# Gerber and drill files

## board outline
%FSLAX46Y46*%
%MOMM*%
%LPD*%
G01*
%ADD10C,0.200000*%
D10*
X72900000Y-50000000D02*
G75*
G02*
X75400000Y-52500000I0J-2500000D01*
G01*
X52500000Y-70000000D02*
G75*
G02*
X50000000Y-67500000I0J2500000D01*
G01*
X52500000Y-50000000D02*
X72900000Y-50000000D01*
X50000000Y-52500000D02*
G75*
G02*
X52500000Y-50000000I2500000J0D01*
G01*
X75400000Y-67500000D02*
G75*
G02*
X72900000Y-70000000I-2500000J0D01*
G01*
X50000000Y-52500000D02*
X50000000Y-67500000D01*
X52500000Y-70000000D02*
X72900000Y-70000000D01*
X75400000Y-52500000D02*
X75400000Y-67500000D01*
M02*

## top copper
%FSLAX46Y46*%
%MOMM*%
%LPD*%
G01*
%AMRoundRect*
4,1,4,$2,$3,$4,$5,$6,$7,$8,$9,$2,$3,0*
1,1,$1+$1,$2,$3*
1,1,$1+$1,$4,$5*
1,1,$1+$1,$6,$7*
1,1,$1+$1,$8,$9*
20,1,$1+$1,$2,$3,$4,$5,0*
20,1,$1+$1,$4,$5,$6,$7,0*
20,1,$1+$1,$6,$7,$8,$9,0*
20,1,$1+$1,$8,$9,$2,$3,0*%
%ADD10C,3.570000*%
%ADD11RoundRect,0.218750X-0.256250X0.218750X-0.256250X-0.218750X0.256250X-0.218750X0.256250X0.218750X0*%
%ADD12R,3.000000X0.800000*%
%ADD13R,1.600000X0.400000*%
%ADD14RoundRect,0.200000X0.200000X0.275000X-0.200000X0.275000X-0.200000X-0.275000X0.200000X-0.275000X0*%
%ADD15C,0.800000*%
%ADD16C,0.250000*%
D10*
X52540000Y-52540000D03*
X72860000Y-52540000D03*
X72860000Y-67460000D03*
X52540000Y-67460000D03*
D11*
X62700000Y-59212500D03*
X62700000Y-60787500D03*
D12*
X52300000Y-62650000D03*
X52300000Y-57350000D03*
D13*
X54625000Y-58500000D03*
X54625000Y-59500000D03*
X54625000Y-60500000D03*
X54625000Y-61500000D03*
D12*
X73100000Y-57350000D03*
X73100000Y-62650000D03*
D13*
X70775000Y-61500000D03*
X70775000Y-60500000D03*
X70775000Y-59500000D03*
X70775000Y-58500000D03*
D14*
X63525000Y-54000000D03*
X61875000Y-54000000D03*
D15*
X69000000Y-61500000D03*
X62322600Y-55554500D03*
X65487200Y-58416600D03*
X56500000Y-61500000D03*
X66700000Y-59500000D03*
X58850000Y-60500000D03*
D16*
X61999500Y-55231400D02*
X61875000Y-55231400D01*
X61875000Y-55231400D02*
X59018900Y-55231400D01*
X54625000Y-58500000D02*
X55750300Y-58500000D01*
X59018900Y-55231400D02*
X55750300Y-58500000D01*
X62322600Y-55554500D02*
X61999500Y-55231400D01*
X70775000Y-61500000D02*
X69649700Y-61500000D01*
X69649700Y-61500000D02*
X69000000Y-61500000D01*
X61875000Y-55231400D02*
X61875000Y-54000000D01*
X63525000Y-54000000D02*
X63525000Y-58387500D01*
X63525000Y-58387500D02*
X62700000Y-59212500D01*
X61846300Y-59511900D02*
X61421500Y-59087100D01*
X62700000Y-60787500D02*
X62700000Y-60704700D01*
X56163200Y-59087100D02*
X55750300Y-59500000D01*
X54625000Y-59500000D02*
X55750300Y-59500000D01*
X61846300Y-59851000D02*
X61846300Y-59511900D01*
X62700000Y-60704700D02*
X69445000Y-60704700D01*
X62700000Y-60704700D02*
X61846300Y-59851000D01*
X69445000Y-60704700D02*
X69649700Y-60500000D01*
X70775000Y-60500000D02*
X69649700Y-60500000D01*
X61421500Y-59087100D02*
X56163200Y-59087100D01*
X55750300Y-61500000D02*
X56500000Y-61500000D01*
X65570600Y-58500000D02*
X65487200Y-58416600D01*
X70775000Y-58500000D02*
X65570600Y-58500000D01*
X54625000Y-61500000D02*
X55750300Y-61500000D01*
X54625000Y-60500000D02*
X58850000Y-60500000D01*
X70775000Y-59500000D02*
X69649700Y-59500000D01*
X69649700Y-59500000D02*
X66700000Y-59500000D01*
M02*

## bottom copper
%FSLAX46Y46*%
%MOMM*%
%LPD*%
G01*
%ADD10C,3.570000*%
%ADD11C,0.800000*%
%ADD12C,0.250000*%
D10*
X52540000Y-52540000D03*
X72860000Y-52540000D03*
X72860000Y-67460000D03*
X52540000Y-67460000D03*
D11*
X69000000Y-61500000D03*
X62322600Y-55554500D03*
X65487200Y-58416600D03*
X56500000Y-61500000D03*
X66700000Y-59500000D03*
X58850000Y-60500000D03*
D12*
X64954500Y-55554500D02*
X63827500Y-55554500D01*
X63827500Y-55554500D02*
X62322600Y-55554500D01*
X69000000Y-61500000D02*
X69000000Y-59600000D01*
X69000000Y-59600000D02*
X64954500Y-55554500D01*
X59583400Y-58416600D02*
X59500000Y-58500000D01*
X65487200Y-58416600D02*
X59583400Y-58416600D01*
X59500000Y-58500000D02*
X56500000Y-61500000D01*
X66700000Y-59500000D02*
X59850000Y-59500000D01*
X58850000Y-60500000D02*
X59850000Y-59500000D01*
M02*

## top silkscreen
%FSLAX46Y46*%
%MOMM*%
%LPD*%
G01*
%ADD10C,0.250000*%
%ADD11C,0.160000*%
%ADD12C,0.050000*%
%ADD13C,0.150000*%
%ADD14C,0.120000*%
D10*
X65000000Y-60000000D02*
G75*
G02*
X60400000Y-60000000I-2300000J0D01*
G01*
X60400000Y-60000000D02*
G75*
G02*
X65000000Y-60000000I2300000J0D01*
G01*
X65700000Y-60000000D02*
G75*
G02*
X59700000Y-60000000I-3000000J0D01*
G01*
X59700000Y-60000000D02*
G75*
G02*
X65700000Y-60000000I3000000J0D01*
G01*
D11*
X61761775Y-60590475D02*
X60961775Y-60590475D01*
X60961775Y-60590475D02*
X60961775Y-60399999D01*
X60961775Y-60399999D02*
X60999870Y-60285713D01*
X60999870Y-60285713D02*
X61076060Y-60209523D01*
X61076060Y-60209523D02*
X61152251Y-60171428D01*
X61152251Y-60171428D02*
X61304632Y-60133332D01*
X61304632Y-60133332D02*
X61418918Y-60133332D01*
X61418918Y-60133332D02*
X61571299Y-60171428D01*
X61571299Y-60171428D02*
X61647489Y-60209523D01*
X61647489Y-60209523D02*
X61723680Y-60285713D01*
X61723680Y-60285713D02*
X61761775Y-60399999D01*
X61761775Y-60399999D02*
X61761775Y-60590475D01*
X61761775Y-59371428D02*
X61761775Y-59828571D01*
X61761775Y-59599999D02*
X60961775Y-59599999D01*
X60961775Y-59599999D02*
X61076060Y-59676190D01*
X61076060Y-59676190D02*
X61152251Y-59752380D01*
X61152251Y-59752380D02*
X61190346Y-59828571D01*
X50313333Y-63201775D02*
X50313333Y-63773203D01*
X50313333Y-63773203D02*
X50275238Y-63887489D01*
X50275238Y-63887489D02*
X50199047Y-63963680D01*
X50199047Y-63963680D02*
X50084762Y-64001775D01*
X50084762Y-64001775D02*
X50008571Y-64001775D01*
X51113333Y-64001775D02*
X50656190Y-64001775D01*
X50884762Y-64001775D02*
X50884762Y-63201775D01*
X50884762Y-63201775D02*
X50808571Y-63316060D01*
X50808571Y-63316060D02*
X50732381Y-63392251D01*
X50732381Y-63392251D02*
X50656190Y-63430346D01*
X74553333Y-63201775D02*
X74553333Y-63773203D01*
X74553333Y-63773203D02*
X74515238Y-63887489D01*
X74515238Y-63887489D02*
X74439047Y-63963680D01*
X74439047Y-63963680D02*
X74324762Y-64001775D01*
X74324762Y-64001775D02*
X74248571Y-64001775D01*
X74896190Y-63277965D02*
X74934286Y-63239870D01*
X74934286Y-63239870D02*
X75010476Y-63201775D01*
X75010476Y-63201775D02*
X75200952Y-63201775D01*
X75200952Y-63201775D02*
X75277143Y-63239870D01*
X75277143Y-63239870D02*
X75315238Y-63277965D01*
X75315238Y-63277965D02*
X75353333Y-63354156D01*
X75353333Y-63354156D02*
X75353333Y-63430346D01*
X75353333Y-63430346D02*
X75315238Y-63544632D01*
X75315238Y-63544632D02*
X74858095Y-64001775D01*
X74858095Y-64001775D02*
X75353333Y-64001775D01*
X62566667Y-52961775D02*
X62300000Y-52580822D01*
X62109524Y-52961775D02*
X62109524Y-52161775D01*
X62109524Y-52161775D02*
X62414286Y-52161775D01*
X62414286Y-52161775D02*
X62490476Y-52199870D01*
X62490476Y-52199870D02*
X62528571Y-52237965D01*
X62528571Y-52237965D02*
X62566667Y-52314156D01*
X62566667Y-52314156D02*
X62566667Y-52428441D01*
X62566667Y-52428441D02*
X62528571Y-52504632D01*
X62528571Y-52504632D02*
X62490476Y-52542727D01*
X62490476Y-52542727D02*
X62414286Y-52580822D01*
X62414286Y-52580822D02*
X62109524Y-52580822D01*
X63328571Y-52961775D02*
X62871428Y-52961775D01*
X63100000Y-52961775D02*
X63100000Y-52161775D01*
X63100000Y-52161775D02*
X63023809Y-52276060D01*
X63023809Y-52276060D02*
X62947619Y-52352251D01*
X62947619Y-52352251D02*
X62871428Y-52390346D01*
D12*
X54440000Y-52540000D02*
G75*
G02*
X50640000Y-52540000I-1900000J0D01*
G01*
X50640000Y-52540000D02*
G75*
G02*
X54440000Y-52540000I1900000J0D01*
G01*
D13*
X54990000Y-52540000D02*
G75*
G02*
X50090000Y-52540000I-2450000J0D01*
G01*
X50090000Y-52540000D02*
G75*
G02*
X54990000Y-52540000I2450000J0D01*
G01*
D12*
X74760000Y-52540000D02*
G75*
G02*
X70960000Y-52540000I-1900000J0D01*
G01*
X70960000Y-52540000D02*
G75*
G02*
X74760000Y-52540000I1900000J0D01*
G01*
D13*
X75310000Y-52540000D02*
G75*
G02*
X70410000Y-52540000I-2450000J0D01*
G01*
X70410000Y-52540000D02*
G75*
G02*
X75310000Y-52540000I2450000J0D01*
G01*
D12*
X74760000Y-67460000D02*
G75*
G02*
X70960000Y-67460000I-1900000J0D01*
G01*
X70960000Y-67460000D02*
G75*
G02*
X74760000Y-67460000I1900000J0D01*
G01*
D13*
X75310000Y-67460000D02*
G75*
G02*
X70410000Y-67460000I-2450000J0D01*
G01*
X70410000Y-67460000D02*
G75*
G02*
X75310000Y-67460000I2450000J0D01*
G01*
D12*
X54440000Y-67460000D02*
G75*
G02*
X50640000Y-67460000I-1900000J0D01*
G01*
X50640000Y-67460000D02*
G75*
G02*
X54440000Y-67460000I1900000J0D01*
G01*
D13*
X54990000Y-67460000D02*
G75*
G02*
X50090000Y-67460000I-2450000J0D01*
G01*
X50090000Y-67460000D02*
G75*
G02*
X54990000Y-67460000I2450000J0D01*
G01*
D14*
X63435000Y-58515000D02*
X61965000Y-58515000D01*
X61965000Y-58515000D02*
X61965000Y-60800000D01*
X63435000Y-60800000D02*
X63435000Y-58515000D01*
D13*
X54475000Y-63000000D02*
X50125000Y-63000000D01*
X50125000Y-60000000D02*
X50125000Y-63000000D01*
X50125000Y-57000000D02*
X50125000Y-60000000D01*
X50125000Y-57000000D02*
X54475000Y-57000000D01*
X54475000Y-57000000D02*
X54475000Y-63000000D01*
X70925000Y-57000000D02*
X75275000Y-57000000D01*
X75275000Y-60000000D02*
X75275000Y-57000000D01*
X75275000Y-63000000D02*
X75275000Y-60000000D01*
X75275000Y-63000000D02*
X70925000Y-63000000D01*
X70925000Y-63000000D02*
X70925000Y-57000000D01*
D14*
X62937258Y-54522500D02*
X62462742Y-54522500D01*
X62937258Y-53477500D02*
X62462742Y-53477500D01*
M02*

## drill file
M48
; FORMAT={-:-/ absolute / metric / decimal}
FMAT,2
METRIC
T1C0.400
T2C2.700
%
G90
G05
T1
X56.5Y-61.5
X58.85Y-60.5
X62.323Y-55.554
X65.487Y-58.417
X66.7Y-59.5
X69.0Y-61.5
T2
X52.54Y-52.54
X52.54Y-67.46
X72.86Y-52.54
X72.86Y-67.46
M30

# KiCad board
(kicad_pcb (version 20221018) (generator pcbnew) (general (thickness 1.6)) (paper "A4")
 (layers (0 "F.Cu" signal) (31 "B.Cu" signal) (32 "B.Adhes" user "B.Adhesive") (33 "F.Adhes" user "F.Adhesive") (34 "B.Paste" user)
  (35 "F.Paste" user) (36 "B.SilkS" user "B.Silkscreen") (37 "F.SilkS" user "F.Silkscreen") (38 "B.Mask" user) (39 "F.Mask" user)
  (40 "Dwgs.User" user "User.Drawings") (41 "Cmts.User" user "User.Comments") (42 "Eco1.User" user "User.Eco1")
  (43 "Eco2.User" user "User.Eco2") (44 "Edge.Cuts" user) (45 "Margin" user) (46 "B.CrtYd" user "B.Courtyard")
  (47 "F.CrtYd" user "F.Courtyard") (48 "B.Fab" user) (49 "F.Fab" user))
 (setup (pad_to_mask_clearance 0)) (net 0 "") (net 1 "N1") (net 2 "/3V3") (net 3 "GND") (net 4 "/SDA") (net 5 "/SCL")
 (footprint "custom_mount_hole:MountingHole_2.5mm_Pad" (layer "F.Cu") (at 52.54 52.54)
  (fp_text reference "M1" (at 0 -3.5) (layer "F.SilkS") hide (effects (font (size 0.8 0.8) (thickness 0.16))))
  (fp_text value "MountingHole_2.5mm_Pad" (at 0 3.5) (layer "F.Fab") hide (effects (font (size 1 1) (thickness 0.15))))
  (fp_circle (center 0 0) (end 1.9 0) (stroke (width 0.05) (type solid)) (fill none) (layer "F.SilkS"))
  (fp_circle (center 0 0) (end 2.45 0) (stroke (width 0.15) (type solid)) (fill none) (layer "F.SilkS"))
  (pad "~" thru_hole circle (at 0 0) (size 3.57 3.57) (drill 2.7) (layers "*.Cu" "*.Mask")))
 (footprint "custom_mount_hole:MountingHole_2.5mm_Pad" (layer "F.Cu") (at 72.86 52.54)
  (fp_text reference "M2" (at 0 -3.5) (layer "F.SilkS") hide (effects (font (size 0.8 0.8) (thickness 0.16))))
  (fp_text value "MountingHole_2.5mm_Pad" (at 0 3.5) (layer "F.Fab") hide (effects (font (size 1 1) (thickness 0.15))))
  (fp_circle (center 0 0) (end 1.9 0) (stroke (width 0.05) (type solid)) (fill none) (layer "F.SilkS"))
  (fp_circle (center 0 0) (end 2.45 0) (stroke (width 0.15) (type solid)) (fill none) (layer "F.SilkS"))
  (pad "~" thru_hole circle (at 0 0) (size 3.57 3.57) (drill 2.7) (layers "*.Cu" "*.Mask")))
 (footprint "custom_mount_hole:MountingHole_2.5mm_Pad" (layer "F.Cu") (at 72.86 67.46)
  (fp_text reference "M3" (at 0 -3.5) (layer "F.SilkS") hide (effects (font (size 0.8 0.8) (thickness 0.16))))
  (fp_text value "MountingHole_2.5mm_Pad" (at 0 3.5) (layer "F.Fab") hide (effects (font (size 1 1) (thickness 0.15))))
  (fp_circle (center 0 0) (end 1.9 0) (stroke (width 0.05) (type solid)) (fill none) (layer "F.SilkS"))
  (fp_circle (center 0 0) (end 2.45 0) (stroke (width 0.15) (type solid)) (fill none) (layer "F.SilkS"))
  (pad "~" thru_hole circle (at 0 0) (size 3.57 3.57) (drill 2.7) (layers "*.Cu" "*.Mask")))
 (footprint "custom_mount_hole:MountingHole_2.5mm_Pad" (layer "F.Cu") (at 52.54 67.46)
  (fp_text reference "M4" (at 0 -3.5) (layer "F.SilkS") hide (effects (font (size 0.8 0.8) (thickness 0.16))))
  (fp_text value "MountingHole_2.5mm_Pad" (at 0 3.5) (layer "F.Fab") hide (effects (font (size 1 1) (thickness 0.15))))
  (fp_circle (center 0 0) (end 1.9 0) (stroke (width 0.05) (type solid)) (fill none) (layer "F.SilkS"))
  (fp_circle (center 0 0) (end 2.45 0) (stroke (width 0.15) (type solid)) (fill none) (layer "F.SilkS"))
  (pad "~" thru_hole circle (at 0 0) (size 3.57 3.57) (drill 2.7) (layers "*.Cu" "*.Mask")))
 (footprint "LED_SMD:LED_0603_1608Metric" (layer "F.Cu") (at 62.7 60 -90)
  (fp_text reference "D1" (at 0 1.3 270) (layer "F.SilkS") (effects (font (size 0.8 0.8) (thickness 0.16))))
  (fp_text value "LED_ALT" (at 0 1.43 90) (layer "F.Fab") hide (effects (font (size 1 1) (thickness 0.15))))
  (fp_line (start -1.485 -0.735) (end -1.485 0.735) (stroke (width 0.12) (type solid)) (layer "F.SilkS"))
  (fp_line (start -1.485 0.735) (end 0.8 0.735) (stroke (width 0.12) (type solid)) (layer "F.SilkS"))
  (fp_line (start 0.8 -0.735) (end -1.485 -0.735) (stroke (width 0.12) (type solid)) (layer "F.SilkS"))
  (pad "1" smd roundrect (at -0.7875 0 270) (size 0.875 0.95) (layers "F.Cu" "F.Paste" "F.Mask") (roundrect_rratio 0.25) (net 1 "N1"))
  (pad "2" smd roundrect (at 0.7875 0 270) (size 0.875 0.95) (layers "F.Cu" "F.Paste" "F.Mask") (roundrect_rratio 0.25) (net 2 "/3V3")))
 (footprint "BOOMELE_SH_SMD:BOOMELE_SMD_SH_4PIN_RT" (layer "F.Cu") (at 52.78 60 90)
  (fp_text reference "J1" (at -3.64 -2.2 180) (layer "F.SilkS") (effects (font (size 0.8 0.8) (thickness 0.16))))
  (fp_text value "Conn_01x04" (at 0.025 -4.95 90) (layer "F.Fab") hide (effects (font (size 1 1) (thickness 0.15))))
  (fp_line (start -3 1.695) (end -3 -2.655) (stroke (width 0.15) (type solid)) (layer "F.SilkS"))
  (fp_line (start 0 -2.655) (end -3 -2.655) (stroke (width 0.15) (type solid)) (layer "F.SilkS"))
  (fp_line (start 3 -2.655) (end 0 -2.655) (stroke (width 0.15) (type solid)) (layer "F.SilkS"))
  (fp_line (start 3 -2.655) (end 3 1.695) (stroke (width 0.15) (type solid)) (layer "F.SilkS"))
  (fp_line (start 3 1.695) (end -3 1.695) (stroke (width 0.15) (type solid)) (layer "F.SilkS"))
  (pad "" smd rect (at -2.65 -0.48 270) (size 0.8 3) (layers "F.Cu" "F.Paste" "F.Mask"))
  (pad "" smd rect (at 2.65 -0.48 270) (size 0.8 3) (layers "F.Cu" "F.Paste" "F.Mask"))
  (pad "1" smd rect (at 1.5 1.845 270) (size 0.4 1.6) (layers "F.Cu" "F.Paste" "F.Mask") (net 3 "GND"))
  (pad "2" smd rect (at 0.5 1.845 270) (size 0.4 1.6) (layers "F.Cu" "F.Paste" "F.Mask") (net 2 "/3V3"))
  (pad "3" smd rect (at -0.5 1.845 270) (size 0.4 1.6) (layers "F.Cu" "F.Paste" "F.Mask") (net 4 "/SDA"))
  (pad "4" smd rect (at -1.5 1.845 270) (size 0.4 1.6) (layers "F.Cu" "F.Paste" "F.Mask") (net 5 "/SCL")))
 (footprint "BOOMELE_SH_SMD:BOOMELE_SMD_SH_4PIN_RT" (layer "F.Cu") (at 72.62 60 -90)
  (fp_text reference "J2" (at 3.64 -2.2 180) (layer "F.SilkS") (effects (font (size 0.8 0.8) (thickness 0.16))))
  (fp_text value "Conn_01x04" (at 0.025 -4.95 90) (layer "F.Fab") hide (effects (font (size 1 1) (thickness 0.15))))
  (fp_line (start -3 1.695) (end -3 -2.655) (stroke (width 0.15) (type solid)) (layer "F.SilkS"))
  (fp_line (start 0 -2.655) (end -3 -2.655) (stroke (width 0.15) (type solid)) (layer "F.SilkS"))
  (fp_line (start 3 -2.655) (end 0 -2.655) (stroke (width 0.15) (type solid)) (layer "F.SilkS"))
  (fp_line (start 3 -2.655) (end 3 1.695) (stroke (width 0.15) (type solid)) (layer "F.SilkS"))
  (fp_line (start 3 1.695) (end -3 1.695) (stroke (width 0.15) (type solid)) (layer "F.SilkS"))
  (pad "" smd rect (at -2.65 -0.48 90) (size 0.8 3) (layers "F.Cu" "F.Paste" "F.Mask"))
  (pad "" smd rect (at 2.65 -0.48 90) (size 0.8 3) (layers "F.Cu" "F.Paste" "F.Mask"))
  (pad "1" smd rect (at 1.5 1.845 90) (size 0.4 1.6) (layers "F.Cu" "F.Paste" "F.Mask") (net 3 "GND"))
  (pad "2" smd rect (at 0.5 1.845 90) (size 0.4 1.6) (layers "F.Cu" "F.Paste" "F.Mask") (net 2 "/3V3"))
  (pad "3" smd rect (at -0.5 1.845 90) (size 0.4 1.6) (layers "F.Cu" "F.Paste" "F.Mask") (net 4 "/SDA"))
  (pad "4" smd rect (at -1.5 1.845 90) (size 0.4 1.6) (layers "F.Cu" "F.Paste" "F.Mask") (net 5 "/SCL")))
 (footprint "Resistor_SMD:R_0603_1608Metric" (layer "F.Cu") (at 62.7 54 180)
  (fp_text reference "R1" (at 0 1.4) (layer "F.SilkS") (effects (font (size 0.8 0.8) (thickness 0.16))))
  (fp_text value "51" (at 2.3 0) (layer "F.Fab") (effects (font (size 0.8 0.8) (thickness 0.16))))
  (fp_line (start -0.237258 -0.5225) (end 0.237258 -0.5225) (stroke (width 0.12) (type solid)) (layer "F.SilkS"))
  (fp_line (start -0.237258 0.5225) (end 0.237258 0.5225) (stroke (width 0.12) (type solid)) (layer "F.SilkS"))
  (pad "1" smd roundrect (at -0.825 0 180) (size 0.8 0.95) (layers "F.Cu" "F.Paste" "F.Mask") (roundrect_rratio 0.25) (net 1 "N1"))
  (pad "2" smd roundrect (at 0.825 0 180) (size 0.8 0.95) (layers "F.Cu" "F.Paste" "F.Mask") (roundrect_rratio 0.25) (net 3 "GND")))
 (gr_circle (center 62.7 60) (end 65 60) (stroke (width 0.25) (type solid)) (fill none) (layer "F.SilkS"))
 (gr_circle (center 62.7 60) (end 65.7 60) (stroke (width 0.25) (type solid)) (fill none) (layer "F.SilkS"))
 (gr_arc (start 72.9 50) (mid 74.667767 50.732233) (end 75.4 52.5) (stroke (width 0.2) (type solid)) (layer "Edge.Cuts"))
 (gr_arc (start 52.5 70) (mid 50.732233 69.267767) (end 50 67.5) (stroke (width 0.2) (type solid)) (layer "Edge.Cuts"))
 (gr_line (start 52.5 50) (end 72.9 50) (stroke (width 0.2) (type solid)) (layer "Edge.Cuts"))
 (gr_arc (start 50 52.5) (mid 50.732233 50.732233) (end 52.5 50) (stroke (width 0.2) (type solid)) (layer "Edge.Cuts"))
 (gr_arc (start 75.4 67.5) (mid 74.667767 69.267767) (end 72.9 70) (stroke (width 0.2) (type solid)) (layer "Edge.Cuts"))
 (gr_line (start 50 52.5) (end 50 67.5) (stroke (width 0.2) (type solid)) (layer "Edge.Cuts"))
 (gr_line (start 52.5 70) (end 72.9 70) (stroke (width 0.2) (type solid)) (layer "Edge.Cuts"))
 (gr_line (start 75.4 52.5) (end 75.4 67.5) (stroke (width 0.2) (type solid)) (layer "Edge.Cuts"))
 (segment (start 61.9995 55.2314) (end 61.875 55.2314) (width 0.25) (layer "F.Cu") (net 3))
 (segment (start 61.875 55.2314) (end 59.0189 55.2314) (width 0.25) (layer "F.Cu") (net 3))
 (segment (start 54.625 58.5) (end 55.7503 58.5) (width 0.25) (layer "F.Cu") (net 3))
 (segment (start 59.0189 55.2314) (end 55.7503 58.5) (width 0.25) (layer "F.Cu") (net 3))
 (segment (start 62.3226 55.5545) (end 61.9995 55.2314) (width 0.25) (layer "F.Cu") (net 3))
 (segment (start 70.775 61.5) (end 69.6497 61.5) (width 0.25) (layer "F.Cu") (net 3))
 (segment (start 69.6497 61.5) (end 69 61.5) (width 0.25) (layer "F.Cu") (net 3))
 (segment (start 61.875 55.2314) (end 61.875 54) (width 0.25) (layer "F.Cu") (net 3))
 (via (at 69 61.5) (size 0.8) (drill 0.4) (layers "F.Cu" "B.Cu") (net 3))
 (via (at 62.3226 55.5545) (size 0.8) (drill 0.4) (layers "F.Cu" "B.Cu") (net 3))
 (segment (start 64.9545 55.5545) (end 63.8275 55.5545) (width 0.25) (layer "B.Cu") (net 3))
 (segment (start 63.8275 55.5545) (end 62.3226 55.5545) (width 0.25) (layer "B.Cu") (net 3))
 (segment (start 69 61.5) (end 69 59.6) (width 0.25) (layer "B.Cu") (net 3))
 (segment (start 69 59.6) (end 64.9545 55.5545) (width 0.25) (layer "B.Cu") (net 3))
 (segment (start 63.525 54) (end 63.525 58.3875) (width 0.25) (layer "F.Cu") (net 1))
 (segment (start 63.525 58.3875) (end 62.7 59.2125) (width 0.25) (layer "F.Cu") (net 1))
 (segment (start 61.8463 59.5119) (end 61.4215 59.0871) (width 0.25) (layer "F.Cu") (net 2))
 (segment (start 62.7 60.7875) (end 62.7 60.7047) (width 0.25) (layer "F.Cu") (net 2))
 (segment (start 56.1632 59.0871) (end 55.7503 59.5) (width 0.25) (layer "F.Cu") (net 2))
 (segment (start 54.625 59.5) (end 55.7503 59.5) (width 0.25) (layer "F.Cu") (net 2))
 (segment (start 61.8463 59.851) (end 61.8463 59.5119) (width 0.25) (layer "F.Cu") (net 2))
 (segment (start 62.7 60.7047) (end 69.445 60.7047) (width 0.25) (layer "F.Cu") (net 2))
 (segment (start 62.7 60.7047) (end 61.8463 59.851) (width 0.25) (layer "F.Cu") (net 2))
 (segment (start 69.445 60.7047) (end 69.6497 60.5) (width 0.25) (layer "F.Cu") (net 2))
 (segment (start 70.775 60.5) (end 69.6497 60.5) (width 0.25) (layer "F.Cu") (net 2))
 (segment (start 61.4215 59.0871) (end 56.1632 59.0871) (width 0.25) (layer "F.Cu") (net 2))
 (segment (start 55.7503 61.5) (end 56.5 61.5) (width 0.25) (layer "F.Cu") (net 5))
 (segment (start 65.5706 58.5) (end 65.4872 58.4166) (width 0.25) (layer "F.Cu") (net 5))
 (segment (start 70.775 58.5) (end 65.5706 58.5) (width 0.25) (layer "F.Cu") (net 5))
 (segment (start 54.625 61.5) (end 55.7503 61.5) (width 0.25) (layer "F.Cu") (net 5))
 (via (at 65.4872 58.4166) (size 0.8) (drill 0.4) (layers "F.Cu" "B.Cu") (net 5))
 (via (at 56.5 61.5) (size 0.8) (drill 0.4) (layers "F.Cu" "B.Cu") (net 5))
 (segment (start 59.5834 58.4166) (end 59.5 58.5) (width 0.25) (layer "B.Cu") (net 5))
 (segment (start 65.4872 58.4166) (end 59.5834 58.4166) (width 0.25) (layer "B.Cu") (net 5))
 (segment (start 59.5 58.5) (end 56.5 61.5) (width 0.25) (layer "B.Cu") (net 5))
 (segment (start 54.625 60.5) (end 58.85 60.5) (width 0.25) (layer "F.Cu") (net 4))
 (segment (start 70.775 59.5) (end 69.6497 59.5) (width 0.25) (layer "F.Cu") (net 4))
 (segment (start 69.6497 59.5) (end 66.7 59.5) (width 0.25) (layer "F.Cu") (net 4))
 (via (at 66.7 59.5) (size 0.8) (drill 0.4) (layers "F.Cu" "B.Cu") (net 4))
 (via (at 58.85 60.5) (size 0.8) (drill 0.4) (layers "F.Cu" "B.Cu") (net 4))
 (segment (start 66.7 59.5) (end 59.85 59.5) (width 0.25) (layer "B.Cu") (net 4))
 (segment (start 58.85 60.5) (end 59.85 59.5) (width 0.25) (layer "B.Cu") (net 4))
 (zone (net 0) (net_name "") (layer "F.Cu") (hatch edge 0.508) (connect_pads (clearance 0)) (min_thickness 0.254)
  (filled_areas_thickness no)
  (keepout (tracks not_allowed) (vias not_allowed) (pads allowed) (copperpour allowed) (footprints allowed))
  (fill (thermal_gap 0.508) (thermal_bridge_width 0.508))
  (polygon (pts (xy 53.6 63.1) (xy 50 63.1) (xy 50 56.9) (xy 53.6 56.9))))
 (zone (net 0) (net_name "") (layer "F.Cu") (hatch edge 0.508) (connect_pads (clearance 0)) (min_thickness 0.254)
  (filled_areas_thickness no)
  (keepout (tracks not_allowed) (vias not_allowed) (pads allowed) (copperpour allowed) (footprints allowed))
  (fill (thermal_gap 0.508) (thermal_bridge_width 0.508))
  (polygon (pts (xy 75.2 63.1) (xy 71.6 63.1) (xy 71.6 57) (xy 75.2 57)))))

